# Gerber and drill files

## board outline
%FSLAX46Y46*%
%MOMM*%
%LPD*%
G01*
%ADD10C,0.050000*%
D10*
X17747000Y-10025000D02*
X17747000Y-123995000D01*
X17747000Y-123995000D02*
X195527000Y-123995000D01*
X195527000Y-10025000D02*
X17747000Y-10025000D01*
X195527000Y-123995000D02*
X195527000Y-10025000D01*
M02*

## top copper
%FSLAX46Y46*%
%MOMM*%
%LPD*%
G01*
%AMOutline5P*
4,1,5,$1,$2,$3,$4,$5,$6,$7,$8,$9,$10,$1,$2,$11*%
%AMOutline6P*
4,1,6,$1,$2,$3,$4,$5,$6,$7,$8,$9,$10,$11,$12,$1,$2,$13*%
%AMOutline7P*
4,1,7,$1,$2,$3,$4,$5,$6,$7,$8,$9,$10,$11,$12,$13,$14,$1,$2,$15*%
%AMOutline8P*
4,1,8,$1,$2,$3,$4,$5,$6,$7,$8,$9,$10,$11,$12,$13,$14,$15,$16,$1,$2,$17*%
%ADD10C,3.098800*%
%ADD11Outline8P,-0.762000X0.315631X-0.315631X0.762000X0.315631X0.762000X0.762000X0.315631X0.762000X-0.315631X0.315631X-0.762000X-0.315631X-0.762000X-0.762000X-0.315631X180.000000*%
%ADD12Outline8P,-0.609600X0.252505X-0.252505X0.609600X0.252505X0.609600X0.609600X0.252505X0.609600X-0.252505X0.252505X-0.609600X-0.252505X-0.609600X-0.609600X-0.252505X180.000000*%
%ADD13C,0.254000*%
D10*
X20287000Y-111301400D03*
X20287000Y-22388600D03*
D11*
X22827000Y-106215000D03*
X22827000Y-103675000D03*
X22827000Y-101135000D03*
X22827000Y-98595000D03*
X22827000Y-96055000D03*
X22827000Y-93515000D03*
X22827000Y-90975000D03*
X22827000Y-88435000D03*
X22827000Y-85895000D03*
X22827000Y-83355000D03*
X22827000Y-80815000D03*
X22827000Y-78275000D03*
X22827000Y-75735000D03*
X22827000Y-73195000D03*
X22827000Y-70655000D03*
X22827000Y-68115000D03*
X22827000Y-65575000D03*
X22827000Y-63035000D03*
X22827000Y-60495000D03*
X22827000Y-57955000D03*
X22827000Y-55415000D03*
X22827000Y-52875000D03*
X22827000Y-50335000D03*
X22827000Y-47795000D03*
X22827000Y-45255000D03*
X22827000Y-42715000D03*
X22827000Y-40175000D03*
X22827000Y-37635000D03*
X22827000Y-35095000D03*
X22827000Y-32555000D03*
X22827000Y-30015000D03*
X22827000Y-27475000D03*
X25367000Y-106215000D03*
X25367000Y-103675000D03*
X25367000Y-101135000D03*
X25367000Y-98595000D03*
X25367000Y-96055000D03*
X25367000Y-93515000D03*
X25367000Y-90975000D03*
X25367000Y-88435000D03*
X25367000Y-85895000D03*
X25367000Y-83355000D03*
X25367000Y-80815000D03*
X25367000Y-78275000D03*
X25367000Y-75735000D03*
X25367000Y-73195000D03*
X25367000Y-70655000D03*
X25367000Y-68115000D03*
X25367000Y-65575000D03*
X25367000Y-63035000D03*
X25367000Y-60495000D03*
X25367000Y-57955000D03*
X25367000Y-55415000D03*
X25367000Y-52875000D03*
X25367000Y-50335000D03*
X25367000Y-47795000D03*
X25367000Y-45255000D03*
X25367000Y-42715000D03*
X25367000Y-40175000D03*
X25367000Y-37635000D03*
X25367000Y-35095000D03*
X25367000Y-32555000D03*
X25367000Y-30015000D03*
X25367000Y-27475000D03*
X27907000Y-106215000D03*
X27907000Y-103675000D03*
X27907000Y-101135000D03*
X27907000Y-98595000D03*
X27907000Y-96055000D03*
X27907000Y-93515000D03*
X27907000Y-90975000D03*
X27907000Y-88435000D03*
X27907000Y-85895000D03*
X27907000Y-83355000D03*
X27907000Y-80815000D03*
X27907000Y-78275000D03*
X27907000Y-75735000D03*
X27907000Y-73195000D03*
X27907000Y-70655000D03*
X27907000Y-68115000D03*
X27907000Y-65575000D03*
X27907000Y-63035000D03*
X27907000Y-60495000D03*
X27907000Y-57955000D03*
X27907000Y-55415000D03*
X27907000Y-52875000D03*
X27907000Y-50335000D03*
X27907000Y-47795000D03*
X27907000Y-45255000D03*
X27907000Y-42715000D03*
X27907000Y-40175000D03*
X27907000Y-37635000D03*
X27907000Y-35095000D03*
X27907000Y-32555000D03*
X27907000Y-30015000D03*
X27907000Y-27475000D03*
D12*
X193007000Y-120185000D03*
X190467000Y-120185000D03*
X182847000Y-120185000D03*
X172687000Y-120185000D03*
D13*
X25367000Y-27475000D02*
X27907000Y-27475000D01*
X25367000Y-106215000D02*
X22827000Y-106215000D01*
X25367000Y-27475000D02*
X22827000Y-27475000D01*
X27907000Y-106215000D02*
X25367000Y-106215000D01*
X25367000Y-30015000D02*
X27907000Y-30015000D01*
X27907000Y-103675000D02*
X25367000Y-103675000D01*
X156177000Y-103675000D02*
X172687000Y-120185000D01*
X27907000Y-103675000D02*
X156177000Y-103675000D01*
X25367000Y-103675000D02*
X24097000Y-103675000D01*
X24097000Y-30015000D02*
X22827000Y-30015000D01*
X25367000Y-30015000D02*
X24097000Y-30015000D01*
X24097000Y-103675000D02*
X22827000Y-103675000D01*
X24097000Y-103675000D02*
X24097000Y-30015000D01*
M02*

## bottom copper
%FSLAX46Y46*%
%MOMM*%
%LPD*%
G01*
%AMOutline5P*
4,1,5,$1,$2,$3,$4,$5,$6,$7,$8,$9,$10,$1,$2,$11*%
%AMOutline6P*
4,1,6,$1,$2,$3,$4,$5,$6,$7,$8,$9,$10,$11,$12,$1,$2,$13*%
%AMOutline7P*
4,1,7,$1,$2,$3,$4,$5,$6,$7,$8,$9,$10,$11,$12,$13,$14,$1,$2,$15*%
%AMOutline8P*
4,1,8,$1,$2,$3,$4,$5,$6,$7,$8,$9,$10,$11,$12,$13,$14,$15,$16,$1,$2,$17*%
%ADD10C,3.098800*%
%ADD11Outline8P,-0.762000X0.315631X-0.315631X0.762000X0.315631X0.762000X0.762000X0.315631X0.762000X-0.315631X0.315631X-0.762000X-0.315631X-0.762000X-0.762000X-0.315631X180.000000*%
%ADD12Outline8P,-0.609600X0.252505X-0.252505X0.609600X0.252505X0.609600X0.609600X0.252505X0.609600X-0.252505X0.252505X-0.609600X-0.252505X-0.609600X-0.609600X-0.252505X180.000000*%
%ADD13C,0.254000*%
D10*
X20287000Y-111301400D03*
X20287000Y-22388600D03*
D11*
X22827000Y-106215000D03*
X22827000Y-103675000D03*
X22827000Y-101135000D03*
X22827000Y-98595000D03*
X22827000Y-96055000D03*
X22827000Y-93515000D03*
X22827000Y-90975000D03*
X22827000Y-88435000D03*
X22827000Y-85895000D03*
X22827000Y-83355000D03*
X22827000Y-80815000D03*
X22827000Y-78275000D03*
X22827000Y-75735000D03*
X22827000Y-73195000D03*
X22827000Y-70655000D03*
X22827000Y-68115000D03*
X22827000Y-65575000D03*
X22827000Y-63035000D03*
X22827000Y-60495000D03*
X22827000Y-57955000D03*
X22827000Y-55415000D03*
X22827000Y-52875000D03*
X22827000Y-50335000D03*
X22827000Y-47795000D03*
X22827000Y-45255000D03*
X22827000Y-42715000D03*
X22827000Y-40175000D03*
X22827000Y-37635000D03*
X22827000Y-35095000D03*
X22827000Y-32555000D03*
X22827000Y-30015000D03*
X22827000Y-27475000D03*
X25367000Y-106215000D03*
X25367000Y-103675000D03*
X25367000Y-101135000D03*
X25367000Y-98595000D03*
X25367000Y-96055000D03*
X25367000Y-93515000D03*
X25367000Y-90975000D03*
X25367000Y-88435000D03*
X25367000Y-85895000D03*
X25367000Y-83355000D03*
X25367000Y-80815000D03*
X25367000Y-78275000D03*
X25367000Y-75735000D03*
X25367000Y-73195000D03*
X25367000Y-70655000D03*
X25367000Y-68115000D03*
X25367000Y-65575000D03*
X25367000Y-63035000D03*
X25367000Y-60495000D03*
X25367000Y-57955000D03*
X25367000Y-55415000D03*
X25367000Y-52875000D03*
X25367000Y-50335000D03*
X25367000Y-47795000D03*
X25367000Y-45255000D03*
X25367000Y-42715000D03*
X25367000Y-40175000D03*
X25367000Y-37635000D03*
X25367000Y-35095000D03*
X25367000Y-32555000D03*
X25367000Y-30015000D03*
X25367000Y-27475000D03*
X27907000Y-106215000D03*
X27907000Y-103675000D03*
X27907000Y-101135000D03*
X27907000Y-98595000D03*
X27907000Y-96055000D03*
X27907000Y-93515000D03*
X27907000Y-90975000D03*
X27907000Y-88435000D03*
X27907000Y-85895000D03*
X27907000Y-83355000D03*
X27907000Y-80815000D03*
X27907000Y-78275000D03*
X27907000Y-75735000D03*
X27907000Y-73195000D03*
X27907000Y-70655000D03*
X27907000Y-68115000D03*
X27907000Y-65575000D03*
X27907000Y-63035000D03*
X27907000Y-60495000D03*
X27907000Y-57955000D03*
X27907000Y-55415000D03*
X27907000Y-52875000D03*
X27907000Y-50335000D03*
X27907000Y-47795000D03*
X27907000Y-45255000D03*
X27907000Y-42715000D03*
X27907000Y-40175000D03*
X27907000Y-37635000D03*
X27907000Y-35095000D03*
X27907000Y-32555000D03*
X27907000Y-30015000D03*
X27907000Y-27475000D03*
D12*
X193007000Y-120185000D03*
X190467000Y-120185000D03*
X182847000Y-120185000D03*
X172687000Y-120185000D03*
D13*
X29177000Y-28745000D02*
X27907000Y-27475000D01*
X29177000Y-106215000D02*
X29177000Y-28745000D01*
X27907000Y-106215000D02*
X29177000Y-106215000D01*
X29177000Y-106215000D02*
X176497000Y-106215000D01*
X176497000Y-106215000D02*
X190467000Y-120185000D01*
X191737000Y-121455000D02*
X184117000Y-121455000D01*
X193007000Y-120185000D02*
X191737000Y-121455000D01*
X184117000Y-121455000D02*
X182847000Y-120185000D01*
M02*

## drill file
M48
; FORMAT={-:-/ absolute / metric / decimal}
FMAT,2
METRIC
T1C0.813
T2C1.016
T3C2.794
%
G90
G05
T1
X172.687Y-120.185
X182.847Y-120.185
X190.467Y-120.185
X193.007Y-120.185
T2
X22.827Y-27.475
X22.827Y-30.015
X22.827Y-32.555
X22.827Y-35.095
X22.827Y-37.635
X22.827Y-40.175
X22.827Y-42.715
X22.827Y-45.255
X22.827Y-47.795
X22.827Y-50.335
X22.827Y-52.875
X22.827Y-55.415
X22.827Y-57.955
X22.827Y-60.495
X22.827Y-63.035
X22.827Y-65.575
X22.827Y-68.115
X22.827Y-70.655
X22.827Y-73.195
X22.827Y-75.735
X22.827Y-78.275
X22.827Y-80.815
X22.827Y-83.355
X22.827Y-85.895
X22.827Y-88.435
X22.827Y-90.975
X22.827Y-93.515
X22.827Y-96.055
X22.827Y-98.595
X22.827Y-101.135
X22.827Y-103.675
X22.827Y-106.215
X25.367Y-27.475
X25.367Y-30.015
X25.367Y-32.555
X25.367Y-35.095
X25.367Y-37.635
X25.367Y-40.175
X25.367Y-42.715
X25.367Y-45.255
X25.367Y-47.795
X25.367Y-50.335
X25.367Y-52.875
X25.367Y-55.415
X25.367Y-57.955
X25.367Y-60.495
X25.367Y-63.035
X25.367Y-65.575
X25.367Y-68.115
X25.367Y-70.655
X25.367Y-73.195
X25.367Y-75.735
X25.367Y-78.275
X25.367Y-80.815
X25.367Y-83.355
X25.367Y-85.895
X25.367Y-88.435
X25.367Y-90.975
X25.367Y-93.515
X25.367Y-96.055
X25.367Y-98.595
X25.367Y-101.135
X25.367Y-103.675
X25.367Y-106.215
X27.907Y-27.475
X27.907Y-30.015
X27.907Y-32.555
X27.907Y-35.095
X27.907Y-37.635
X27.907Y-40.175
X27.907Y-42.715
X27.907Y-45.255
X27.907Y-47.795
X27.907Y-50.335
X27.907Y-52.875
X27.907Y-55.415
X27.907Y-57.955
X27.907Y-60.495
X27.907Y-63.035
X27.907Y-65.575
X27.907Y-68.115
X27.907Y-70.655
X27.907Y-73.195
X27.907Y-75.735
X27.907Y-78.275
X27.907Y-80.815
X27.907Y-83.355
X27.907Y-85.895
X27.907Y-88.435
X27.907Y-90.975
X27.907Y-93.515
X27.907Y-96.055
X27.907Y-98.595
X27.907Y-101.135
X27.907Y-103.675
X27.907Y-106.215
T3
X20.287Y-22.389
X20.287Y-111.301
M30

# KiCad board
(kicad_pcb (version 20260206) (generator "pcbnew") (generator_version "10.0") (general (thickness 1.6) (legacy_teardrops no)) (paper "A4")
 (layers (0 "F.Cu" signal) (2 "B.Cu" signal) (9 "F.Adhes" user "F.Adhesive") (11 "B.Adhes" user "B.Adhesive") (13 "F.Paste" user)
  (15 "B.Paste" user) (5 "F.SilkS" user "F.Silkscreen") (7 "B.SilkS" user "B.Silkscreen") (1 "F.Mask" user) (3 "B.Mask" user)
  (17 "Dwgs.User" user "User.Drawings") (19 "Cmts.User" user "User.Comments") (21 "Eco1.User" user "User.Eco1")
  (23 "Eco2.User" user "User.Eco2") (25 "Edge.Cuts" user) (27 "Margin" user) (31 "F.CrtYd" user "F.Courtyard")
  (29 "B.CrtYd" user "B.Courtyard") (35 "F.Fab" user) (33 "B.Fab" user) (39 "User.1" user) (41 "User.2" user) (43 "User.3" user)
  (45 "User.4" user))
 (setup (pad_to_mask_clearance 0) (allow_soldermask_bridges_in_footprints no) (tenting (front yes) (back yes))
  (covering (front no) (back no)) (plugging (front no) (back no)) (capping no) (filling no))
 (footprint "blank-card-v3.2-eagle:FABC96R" (layer "F.Cu") (at 20.287 66.845 180)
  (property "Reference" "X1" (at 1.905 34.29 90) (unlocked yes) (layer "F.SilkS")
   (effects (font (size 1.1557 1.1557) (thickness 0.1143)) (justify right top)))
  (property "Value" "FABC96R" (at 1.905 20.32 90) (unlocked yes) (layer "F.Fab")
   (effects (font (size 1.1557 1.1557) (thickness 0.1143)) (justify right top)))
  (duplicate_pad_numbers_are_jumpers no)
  (pad "" np_thru_hole circle (at 0 -44.4564 180) (size 3.0988 3.0988) (drill 2.794) (layers "*.Cu" "*.Mask"))
  (pad "" np_thru_hole circle (at 0 44.4564 180) (size 3.0988 3.0988) (drill 2.794) (layers "*.Cu" "*.Mask"))
  (pad "A1" thru_hole roundrect (at -2.54 -39.37 180) (size 1.524 1.524) (drill 1.016) (layers "*.Cu" "*.Mask") (remove_unused_layers no)
   (roundrect_rratio 0.25) (chamfer_ratio 0.2928932188) (chamfer top_left top_right bottom_left bottom_right) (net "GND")
   (solder_mask_margin 0.0635) (thermal_bridge_angle 0))
  (pad "A2" thru_hole roundrect (at -2.54 -36.83 180) (size 1.524 1.524) (drill 1.016) (layers "*.Cu" "*.Mask") (remove_unused_layers no)
   (roundrect_rratio 0.25) (chamfer_ratio 0.2928932188) (chamfer top_left top_right bottom_left bottom_right) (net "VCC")
   (solder_mask_margin 0.0635) (thermal_bridge_angle 0))
  (pad "A3" thru_hole roundrect (at -2.54 -34.29 180) (size 1.524 1.524) (drill 1.016) (layers "*.Cu" "*.Mask") (remove_unused_layers no)
   (roundrect_rratio 0.25) (chamfer_ratio 0.2928932188) (chamfer top_left top_right bottom_left bottom_right) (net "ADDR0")
   (solder_mask_margin 0.0635) (thermal_bridge_angle 0))
  (pad "A4" thru_hole roundrect (at -2.54 -31.75 180) (size 1.524 1.524) (drill 1.016) (layers "*.Cu" "*.Mask") (remove_unused_layers no)
   (roundrect_rratio 0.25) (chamfer_ratio 0.2928932188) (chamfer top_left top_right bottom_left bottom_right) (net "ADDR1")
   (solder_mask_margin 0.0635) (thermal_bridge_angle 0))
  (pad "A5" thru_hole roundrect (at -2.54 -29.21 180) (size 1.524 1.524) (drill 1.016) (layers "*.Cu" "*.Mask") (remove_unused_layers no)
   (roundrect_rratio 0.25) (chamfer_ratio 0.2928932188) (chamfer top_left top_right bottom_left bottom_right) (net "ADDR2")
   (solder_mask_margin 0.0635) (thermal_bridge_angle 0))
  (pad "A6" thru_hole roundrect (at -2.54 -26.67 180) (size 1.524 1.524) (drill 1.016) (layers "*.Cu" "*.Mask") (remove_unused_layers no)
   (roundrect_rratio 0.25) (chamfer_ratio 0.2928932188) (chamfer top_left top_right bottom_left bottom_right) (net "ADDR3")
   (solder_mask_margin 0.0635) (thermal_bridge_angle 0))
  (pad "A7" thru_hole roundrect (at -2.54 -24.13 180) (size 1.524 1.524) (drill 1.016) (layers "*.Cu" "*.Mask") (remove_unused_layers no)
   (roundrect_rratio 0.25) (chamfer_ratio 0.2928932188) (chamfer top_left top_right bottom_left bottom_right) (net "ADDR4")
   (solder_mask_margin 0.0635) (thermal_bridge_angle 0))
  (pad "A8" thru_hole roundrect (at -2.54 -21.59 180) (size 1.524 1.524) (drill 1.016) (layers "*.Cu" "*.Mask") (remove_unused_layers no)
   (roundrect_rratio 0.25) (chamfer_ratio 0.2928932188) (chamfer top_left top_right bottom_left bottom_right) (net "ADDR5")
   (solder_mask_margin 0.0635) (thermal_bridge_angle 0))
  (pad "A9" thru_hole roundrect (at -2.54 -19.05 180) (size 1.524 1.524) (drill 1.016) (layers "*.Cu" "*.Mask") (remove_unused_layers no)
   (roundrect_rratio 0.25) (chamfer_ratio 0.2928932188) (chamfer top_left top_right bottom_left bottom_right) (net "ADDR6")
   (solder_mask_margin 0.0635) (thermal_bridge_angle 0))
  (pad "A10" thru_hole roundrect (at -2.54 -16.51 180) (size 1.524 1.524) (drill 1.016) (layers "*.Cu" "*.Mask") (remove_unused_layers no)
   (roundrect_rratio 0.25) (chamfer_ratio 0.2928932188) (chamfer top_left top_right bottom_left bottom_right) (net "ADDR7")
   (solder_mask_margin 0.0635) (thermal_bridge_angle 0))
  (pad "A11" thru_hole roundrect (at -2.54 -13.97 180) (size 1.524 1.524) (drill 1.016) (layers "*.Cu" "*.Mask") (remove_unused_layers no)
   (roundrect_rratio 0.25) (chamfer_ratio 0.2928932188) (chamfer top_left top_right bottom_left bottom_right) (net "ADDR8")
   (solder_mask_margin 0.0635) (thermal_bridge_angle 0))
  (pad "A12" thru_hole roundrect (at -2.54 -11.43 180) (size 1.524 1.524) (drill 1.016) (layers "*.Cu" "*.Mask") (remove_unused_layers no)
   (roundrect_rratio 0.25) (chamfer_ratio 0.2928932188) (chamfer top_left top_right bottom_left bottom_right) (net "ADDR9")
   (solder_mask_margin 0.0635) (thermal_bridge_angle 0))
  (pad "A13" thru_hole roundrect (at -2.54 -8.89 180) (size 1.524 1.524) (drill 1.016) (layers "*.Cu" "*.Mask") (remove_unused_layers no)
   (roundrect_rratio 0.25) (chamfer_ratio 0.2928932188) (chamfer top_left top_right bottom_left bottom_right) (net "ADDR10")
   (solder_mask_margin 0.0635) (thermal_bridge_angle 0))
  (pad "A14" thru_hole roundrect (at -2.54 -6.35 180) (size 1.524 1.524) (drill 1.016) (layers "*.Cu" "*.Mask") (remove_unused_layers no)
   (roundrect_rratio 0.25) (chamfer_ratio 0.2928932188) (chamfer top_left top_right bottom_left bottom_right) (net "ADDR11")
   (solder_mask_margin 0.0635) (thermal_bridge_angle 0))
  (pad "A15" thru_hole roundrect (at -2.54 -3.81 180) (size 1.524 1.524) (drill 1.016) (layers "*.Cu" "*.Mask") (remove_unused_layers no)
   (roundrect_rratio 0.25) (chamfer_ratio 0.2928932188) (chamfer top_left top_right bottom_left bottom_right) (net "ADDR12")
   (solder_mask_margin 0.0635) (thermal_bridge_angle 0))
  (pad "A16" thru_hole roundrect (at -2.54 -1.27 180) (size 1.524 1.524) (drill 1.016) (layers "*.Cu" "*.Mask") (remove_unused_layers no)
   (roundrect_rratio 0.25) (chamfer_ratio 0.2928932188) (chamfer top_left top_right bottom_left bottom_right) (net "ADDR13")
   (solder_mask_margin 0.0635) (thermal_bridge_angle 0))
  (pad "A17" thru_hole roundrect (at -2.54 1.27 180) (size 1.524 1.524) (drill 1.016) (layers "*.Cu" "*.Mask") (remove_unused_layers no)
   (roundrect_rratio 0.25) (chamfer_ratio 0.2928932188) (chamfer top_left top_right bottom_left bottom_right) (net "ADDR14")
   (solder_mask_margin 0.0635) (thermal_bridge_angle 0))
  (pad "A18" thru_hole roundrect (at -2.54 3.81 180) (size 1.524 1.524) (drill 1.016) (layers "*.Cu" "*.Mask") (remove_unused_layers no)
   (roundrect_rratio 0.25) (chamfer_ratio 0.2928932188) (chamfer top_left top_right bottom_left bottom_right) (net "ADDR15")
   (solder_mask_margin 0.0635) (thermal_bridge_angle 0))
  (pad "A19" thru_hole roundrect (at -2.54 6.35 180) (size 1.524 1.524) (drill 1.016) (layers "*.Cu" "*.Mask") (remove_unused_layers no)
   (roundrect_rratio 0.25) (chamfer_ratio 0.2928932188) (chamfer top_left top_right bottom_left bottom_right) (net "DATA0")
   (solder_mask_margin 0.0635) (thermal_bridge_angle 0))
  (pad "A20" thru_hole roundrect (at -2.54 8.89 180) (size 1.524 1.524) (drill 1.016) (layers "*.Cu" "*.Mask") (remove_unused_layers no)
   (roundrect_rratio 0.25) (chamfer_ratio 0.2928932188) (chamfer top_left top_right bottom_left bottom_right) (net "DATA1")
   (solder_mask_margin 0.0635) (thermal_bridge_angle 0))
  (pad "A21" thru_hole roundrect (at -2.54 11.43 180) (size 1.524 1.524) (drill 1.016) (layers "*.Cu" "*.Mask") (remove_unused_layers no)
   (roundrect_rratio 0.25) (chamfer_ratio 0.2928932188) (chamfer top_left top_right bottom_left bottom_right) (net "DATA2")
   (solder_mask_margin 0.0635) (thermal_bridge_angle 0))
  (pad "A22" thru_hole roundrect (at -2.54 13.97 180) (size 1.524 1.524) (drill 1.016) (layers "*.Cu" "*.Mask") (remove_unused_layers no)
   (roundrect_rratio 0.25) (chamfer_ratio 0.2928932188) (chamfer top_left top_right bottom_left bottom_right) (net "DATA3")
   (solder_mask_margin 0.0635) (thermal_bridge_angle 0))
  (pad "A23" thru_hole roundrect (at -2.54 16.51 180) (size 1.524 1.524) (drill 1.016) (layers "*.Cu" "*.Mask") (remove_unused_layers no)
   (roundrect_rratio 0.25) (chamfer_ratio 0.2928932188) (chamfer top_left top_right bottom_left bottom_right) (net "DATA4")
   (solder_mask_margin 0.0635) (thermal_bridge_angle 0))
  (pad "A24" thru_hole roundrect (at -2.54 19.05 180) (size 1.524 1.524) (drill 1.016) (layers "*.Cu" "*.Mask") (remove_unused_layers no)
   (roundrect_rratio 0.25) (chamfer_ratio 0.2928932188) (chamfer top_left top_right bottom_left bottom_right) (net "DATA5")
   (solder_mask_margin 0.0635) (thermal_bridge_angle 0))
  (pad "A25" thru_hole roundrect (at -2.54 21.59 180) (size 1.524 1.524) (drill 1.016) (layers "*.Cu" "*.Mask") (remove_unused_layers no)
   (roundrect_rratio 0.25) (chamfer_ratio 0.2928932188) (chamfer top_left top_right bottom_left bottom_right) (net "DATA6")
   (solder_mask_margin 0.0635) (thermal_bridge_angle 0))
  (pad "A26" thru_hole roundrect (at -2.54 24.13 180) (size 1.524 1.524) (drill 1.016) (layers "*.Cu" "*.Mask") (remove_unused_layers no)
   (roundrect_rratio 0.25) (chamfer_ratio 0.2928932188) (chamfer top_left top_right bottom_left bottom_right) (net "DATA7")
   (solder_mask_margin 0.0635) (thermal_bridge_angle 0))
  (pad "A27" thru_hole roundrect (at -2.54 26.67 180) (size 1.524 1.524) (drill 1.016) (layers "*.Cu" "*.Mask") (remove_unused_layers no)
   (roundrect_rratio 0.25) (chamfer_ratio 0.2928932188) (chamfer top_left top_right bottom_left bottom_right) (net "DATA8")
   (solder_mask_margin 0.0635) (thermal_bridge_angle 0))
  (pad "A28" thru_hole roundrect (at -2.54 29.21 180) (size 1.524 1.524) (drill 1.016) (layers "*.Cu" "*.Mask") (remove_unused_layers no)
   (roundrect_rratio 0.25) (chamfer_ratio 0.2928932188) (chamfer top_left top_right bottom_left bottom_right) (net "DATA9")
   (solder_mask_margin 0.0635) (thermal_bridge_angle 0))
  (pad "A29" thru_hole roundrect (at -2.54 31.75 180) (size 1.524 1.524) (drill 1.016) (layers "*.Cu" "*.Mask") (remove_unused_layers no)
   (roundrect_rratio 0.25) (chamfer_ratio 0.2928932188) (chamfer top_left top_right bottom_left bottom_right) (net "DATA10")
   (solder_mask_margin 0.0635) (thermal_bridge_angle 0))
  (pad "A30" thru_hole roundrect (at -2.54 34.29 180) (size 1.524 1.524) (drill 1.016) (layers "*.Cu" "*.Mask") (remove_unused_layers no)
   (roundrect_rratio 0.25) (chamfer_ratio 0.2928932188) (chamfer top_left top_right bottom_left bottom_right) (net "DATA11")
   (solder_mask_margin 0.0635) (thermal_bridge_angle 0))
  (pad "A31" thru_hole roundrect (at -2.54 36.83 180) (size 1.524 1.524) (drill 1.016) (layers "*.Cu" "*.Mask") (remove_unused_layers no)
   (roundrect_rratio 0.25) (chamfer_ratio 0.2928932188) (chamfer top_left top_right bottom_left bottom_right) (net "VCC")
   (solder_mask_margin 0.0635) (thermal_bridge_angle 0))
  (pad "A32" thru_hole roundrect (at -2.54 39.37 180) (size 1.524 1.524) (drill 1.016) (layers "*.Cu" "*.Mask") (remove_unused_layers no)
   (roundrect_rratio 0.25) (chamfer_ratio 0.2928932188) (chamfer top_left top_right bottom_left bottom_right) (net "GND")
   (solder_mask_margin 0.0635) (thermal_bridge_angle 0))
  (pad "B1" thru_hole roundrect (at -5.08 -39.37 180) (size 1.524 1.524) (drill 1.016) (layers "*.Cu" "*.Mask") (remove_unused_layers no)
   (roundrect_rratio 0.25) (chamfer_ratio 0.2928932188) (chamfer top_left top_right bottom_left bottom_right) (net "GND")
   (solder_mask_margin 0.0635) (thermal_bridge_angle 0))
  (pad "B2" thru_hole roundrect (at -5.08 -36.83 180) (size 1.524 1.524) (drill 1.016) (layers "*.Cu" "*.Mask") (remove_unused_layers no)
   (roundrect_rratio 0.25) (chamfer_ratio 0.2928932188) (chamfer top_left top_right bottom_left bottom_right) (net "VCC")
   (solder_mask_margin 0.0635) (thermal_bridge_angle 0))
  (pad "B3" thru_hole roundrect (at -5.08 -34.29 180) (size 1.524 1.524) (drill 1.016) (layers "*.Cu" "*.Mask") (remove_unused_layers no)
   (roundrect_rratio 0.25) (chamfer_ratio 0.2928932188) (chamfer top_left top_right bottom_left bottom_right) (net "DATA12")
   (solder_mask_margin 0.0635) (thermal_bridge_angle 0))
  (pad "B4" thru_hole roundrect (at -5.08 -31.75 180) (size 1.524 1.524) (drill 1.016) (layers "*.Cu" "*.Mask") (remove_unused_layers no)
   (roundrect_rratio 0.25) (chamfer_ratio 0.2928932188) (chamfer top_left top_right bottom_left bottom_right) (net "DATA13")
   (solder_mask_margin 0.0635) (thermal_bridge_angle 0))
  (pad "B5" thru_hole roundrect (at -5.08 -29.21 180) (size 1.524 1.524) (drill 1.016) (layers "*.Cu" "*.Mask") (remove_unused_layers no)
   (roundrect_rratio 0.25) (chamfer_ratio 0.2928932188) (chamfer top_left top_right bottom_left bottom_right) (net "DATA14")
   (solder_mask_margin 0.0635) (thermal_bridge_angle 0))
  (pad "B6" thru_hole roundrect (at -5.08 -26.67 180) (size 1.524 1.524) (drill 1.016) (layers "*.Cu" "*.Mask") (remove_unused_layers no)
   (roundrect_rratio 0.25) (chamfer_ratio 0.2928932188) (chamfer top_left top_right bottom_left bottom_right) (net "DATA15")
   (solder_mask_margin 0.0635) (thermal_bridge_angle 0))
  (pad "B7" thru_hole roundrect (at -5.08 -24.13 180) (size 1.524 1.524) (drill 1.016) (layers "*.Cu" "*.Mask") (remove_unused_layers no)
   (roundrect_rratio 0.25) (chamfer_ratio 0.2928932188) (chamfer top_left top_right bottom_left bottom_right) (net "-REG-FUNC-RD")
   (solder_mask_margin 0.0635) (thermal_bridge_angle 0))
  (pad "B8" thru_hole roundrect (at -5.08 -21.59 180) (size 1.524 1.524) (drill 1.016) (layers "*.Cu" "*.Mask") (remove_unused_layers no)
   (roundrect_rratio 0.25) (chamfer_ratio 0.2928932188) (chamfer top_left top_right bottom_left bottom_right) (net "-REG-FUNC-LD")
   (solder_mask_margin 0.0635) (thermal_bridge_angle 0))
  (pad "B9" thru_hole roundrect (at -5.08 -19.05 180) (size 1.524 1.524) (drill 1.016) (layers "*.Cu" "*.Mask") (remove_unused_layers no)
   (roundrect_rratio 0.25) (chamfer_ratio 0.2928932188) (chamfer top_left top_right bottom_left bottom_right) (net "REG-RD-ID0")
   (solder_mask_margin 0.0635) (thermal_bridge_angle 0))
  (pad "B10" thru_hole roundrect (at -5.08 -16.51 180) (size 1.524 1.524) (drill 1.016) (layers "*.Cu" "*.Mask") (remove_unused_layers no)
   (roundrect_rratio 0.25) (chamfer_ratio 0.2928932188) (chamfer top_left top_right bottom_left bottom_right) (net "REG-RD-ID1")
   (solder_mask_margin 0.0635) (thermal_bridge_angle 0))
  (pad "B11" thru_hole roundrect (at -5.08 -13.97 180) (size 1.524 1.524) (drill 1.016) (layers "*.Cu" "*.Mask") (remove_unused_layers no)
   (roundrect_rratio 0.25) (chamfer_ratio 0.2928932188) (chamfer top_left top_right bottom_left bottom_right) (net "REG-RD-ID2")
   (solder_mask_margin 0.0635) (thermal_bridge_angle 0))
  (pad "B12" thru_hole roundrect (at -5.08 -11.43 180) (size 1.524 1.524) (drill 1.016) (layers "*.Cu" "*.Mask") (remove_unused_layers no)
   (roundrect_rratio 0.25) (chamfer_ratio 0.2928932188) (chamfer top_left top_right bottom_left bottom_right) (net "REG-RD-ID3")
   (solder_mask_margin 0.0635) (thermal_bridge_angle 0))
  (pad "B13" thru_hole roundrect (at -5.08 -8.89 180) (size 1.524 1.524) (drill 1.016) (layers "*.Cu" "*.Mask") (remove_unused_layers no)
   (roundrect_rratio 0.25) (chamfer_ratio 0.2928932188) (chamfer top_left top_right bottom_left bottom_right) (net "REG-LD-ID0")
   (solder_mask_margin 0.0635) (thermal_bridge_angle 0))
  (pad "B14" thru_hole roundrect (at -5.08 -6.35 180) (size 1.524 1.524) (drill 1.016) (layers "*.Cu" "*.Mask") (remove_unused_layers no)
   (roundrect_rratio 0.25) (chamfer_ratio 0.2928932188) (chamfer top_left top_right bottom_left bottom_right) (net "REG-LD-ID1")
   (solder_mask_margin 0.0635) (thermal_bridge_angle 0))
  (pad "B15" thru_hole roundrect (at -5.08 -3.81 180) (size 1.524 1.524) (drill 1.016) (layers "*.Cu" "*.Mask") (remove_unused_layers no)
   (roundrect_rratio 0.25) (chamfer_ratio 0.2928932188) (chamfer top_left top_right bottom_left bottom_right) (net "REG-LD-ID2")
   (solder_mask_margin 0.0635) (thermal_bridge_angle 0))
  (pad "B16" thru_hole roundrect (at -5.08 -1.27 180) (size 1.524 1.524) (drill 1.016) (layers "*.Cu" "*.Mask") (remove_unused_layers no)
   (roundrect_rratio 0.25) (chamfer_ratio 0.2928932188) (chamfer top_left top_right bottom_left bottom_right) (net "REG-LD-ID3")
   (solder_mask_margin 0.0635) (thermal_bridge_angle 0))
  (pad "B17" thru_hole roundrect (at -5.08 1.27 180) (size 1.524 1.524) (drill 1.016) (layers "*.Cu" "*.Mask") (remove_unused_layers no)
   (roundrect_rratio 0.25) (chamfer_ratio 0.2928932188) (chamfer top_left top_right bottom_left bottom_right) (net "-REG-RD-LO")
   (solder_mask_margin 0.0635) (thermal_bridge_angle 0))
  (pad "B18" thru_hole roundrect (at -5.08 3.81 180) (size 1.524 1.524) (drill 1.016) (layers "*.Cu" "*.Mask") (remove_unused_layers no)
   (roundrect_rratio 0.25) (chamfer_ratio 0.2928932188) (chamfer top_left top_right bottom_left bottom_right) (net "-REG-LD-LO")
   (solder_mask_margin 0.0635) (thermal_bridge_angle 0))
  (pad "B19" thru_hole roundrect (at -5.08 6.35 180) (size 1.524 1.524) (drill 1.016) (layers "*.Cu" "*.Mask") (remove_unused_layers no)
   (roundrect_rratio 0.25) (chamfer_ratio 0.2928932188) (chamfer top_left top_right bottom_left bottom_right) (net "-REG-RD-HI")
   (solder_mask_margin 0.0635) (thermal_bridge_angle 0))
  (pad "B20" thru_hole roundrect (at -5.08 8.89 180) (size 1.524 1.524) (drill 1.016) (layers "*.Cu" "*.Mask") (remove_unused_layers no)
   (roundrect_rratio 0.25) (chamfer_ratio 0.2928932188) (chamfer top_left top_right bottom_left bottom_right) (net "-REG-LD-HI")
   (solder_mask_margin 0.0635) (thermal_bridge_angle 0))
  (pad "B21" thru_hole roundrect (at -5.08 11.43 180) (size 1.524 1.524) (drill 1.016) (layers "*.Cu" "*.Mask") (remove_unused_layers no)
   (roundrect_rratio 0.25) (chamfer_ratio 0.2928932188) (chamfer top_left top_right bottom_left bottom_right) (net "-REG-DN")
   (solder_mask_margin 0.0635) (thermal_bridge_angle 0))
  (pad "B22" thru_hole roundrect (at -5.08 13.97 180) (size 1.524 1.524) (drill 1.016) (layers "*.Cu" "*.Mask") (remove_unused_layers no)
   (roundrect_rratio 0.25) (chamfer_ratio 0.2928932188) (chamfer top_left top_right bottom_left bottom_right) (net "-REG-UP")
   (solder_mask_margin 0.0635) (thermal_bridge_angle 0))
  (pad "B23" thru_hole roundrect (at -5.08 16.51 180) (size 1.524 1.524) (drill 1.016) (layers "*.Cu" "*.Mask") (remove_unused_layers no)
   (roundrect_rratio 0.25) (chamfer_ratio 0.2928932188) (chamfer top_left top_right bottom_left bottom_right) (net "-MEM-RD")
   (solder_mask_margin 0.0635) (thermal_bridge_angle 0))
  (pad "B24" thru_hole roundrect (at -5.08 19.05 180) (size 1.524 1.524) (drill 1.016) (layers "*.Cu" "*.Mask") (remove_unused_layers no)
   (roundrect_rratio 0.25) (chamfer_ratio 0.2928932188) (chamfer top_left top_right bottom_left bottom_right) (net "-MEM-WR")
   (solder_mask_margin 0.0635) (thermal_bridge_angle 0))
  (pad "B25" thru_hole roundrect (at -5.08 21.59 180) (size 1.524 1.524) (drill 1.016) (layers "*.Cu" "*.Mask") (remove_unused_layers no)
   (roundrect_rratio 0.25) (chamfer_ratio 0.2928932188) (chamfer top_left top_right bottom_left bottom_right) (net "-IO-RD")
   (solder_mask_margin 0.0635) (thermal_bridge_angle 0))
  (pad "B26" thru_hole roundrect (at -5.08 24.13 180) (size 1.524 1.524) (drill 1.016) (layers "*.Cu" "*.Mask") (remove_unused_layers no)
   (roundrect_rratio 0.25) (chamfer_ratio 0.2928932188) (chamfer top_left top_right bottom_left bottom_right) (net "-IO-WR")
   (solder_mask_margin 0.0635) (thermal_bridge_angle 0))
  (pad "B27" thru_hole roundrect (at -5.08 26.67 180) (size 1.524 1.524) (drill 1.016) (layers "*.Cu" "*.Mask") (remove_unused_layers no)
   (roundrect_rratio 0.25) (chamfer_ratio 0.2928932188) (chamfer top_left top_right bottom_left bottom_right) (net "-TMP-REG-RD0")
   (solder_mask_margin 0.0635) (thermal_bridge_angle 0))
  (pad "B28" thru_hole roundrect (at -5.08 29.21 180) (size 1.524 1.524) (drill 1.016) (layers "*.Cu" "*.Mask") (remove_unused_layers no)
   (roundrect_rratio 0.25) (chamfer_ratio 0.2928932188) (chamfer top_left top_right bottom_left bottom_right) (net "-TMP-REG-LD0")
   (solder_mask_margin 0.0635) (thermal_bridge_angle 0))
  (pad "B29" thru_hole roundrect (at -5.08 31.75 180) (size 1.524 1.524) (drill 1.016) (layers "*.Cu" "*.Mask") (remove_unused_layers no)
   (roundrect_rratio 0.25) (chamfer_ratio 0.2928932188) (chamfer top_left top_right bottom_left bottom_right) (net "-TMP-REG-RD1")
   (solder_mask_margin 0.0635) (thermal_bridge_angle 0))
  (pad "B30" thru_hole roundrect (at -5.08 34.29 180) (size 1.524 1.524) (drill 1.016) (layers "*.Cu" "*.Mask") (remove_unused_layers no)
   (roundrect_rratio 0.25) (chamfer_ratio 0.2928932188) (chamfer top_left top_right bottom_left bottom_right) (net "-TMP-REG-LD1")
   (solder_mask_margin 0.0635) (thermal_bridge_angle 0))
  (pad "B31" thru_hole roundrect (at -5.08 36.83 180) (size 1.524 1.524) (drill 1.016) (layers "*.Cu" "*.Mask") (remove_unused_layers no)
   (roundrect_rratio 0.25) (chamfer_ratio 0.2928932188) (chamfer top_left top_right bottom_left bottom_right) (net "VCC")
   (solder_mask_margin 0.0635) (thermal_bridge_angle 0))
  (pad "B32" thru_hole roundrect (at -5.08 39.37 180) (size 1.524 1.524) (drill 1.016) (layers "*.Cu" "*.Mask") (remove_unused_layers no)
   (roundrect_rratio 0.25) (chamfer_ratio 0.2928932188) (chamfer top_left top_right bottom_left bottom_right) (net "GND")
   (solder_mask_margin 0.0635) (thermal_bridge_angle 0))
  (pad "C1" thru_hole roundrect (at -7.62 -39.37 180) (size 1.524 1.524) (drill 1.016) (layers "*.Cu" "*.Mask") (remove_unused_layers no)
   (roundrect_rratio 0.25) (chamfer_ratio 0.2928932188) (chamfer top_left top_right bottom_left bottom_right) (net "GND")
   (solder_mask_margin 0.0635) (thermal_bridge_angle 0))
  (pad "C2" thru_hole roundrect (at -7.62 -36.83 180) (size 1.524 1.524) (drill 1.016) (layers "*.Cu" "*.Mask") (remove_unused_layers no)
   (roundrect_rratio 0.25) (chamfer_ratio 0.2928932188) (chamfer top_left top_right bottom_left bottom_right) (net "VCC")
   (solder_mask_margin 0.0635) (thermal_bridge_angle 0))
  (pad "C3" thru_hole roundrect (at -7.62 -34.29 180) (size 1.524 1.524) (drill 1.016) (layers "*.Cu" "*.Mask") (remove_unused_layers no)
   (roundrect_rratio 0.25) (chamfer_ratio 0.2928932188) (chamfer top_left top_right bottom_left bottom_right) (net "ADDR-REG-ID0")
   (solder_mask_margin 0.0635) (thermal_bridge_angle 0))
  (pad "C4" thru_hole roundrect (at -7.62 -31.75 180) (size 1.524 1.524) (drill 1.016) (layers "*.Cu" "*.Mask") (remove_unused_layers no)
   (roundrect_rratio 0.25) (chamfer_ratio 0.2928932188) (chamfer top_left top_right bottom_left bottom_right) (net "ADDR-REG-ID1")
   (solder_mask_margin 0.0635) (thermal_bridge_angle 0))
  (pad "C5" thru_hole roundrect (at -7.62 -29.21 180) (size 1.524 1.524) (drill 1.016) (layers "*.Cu" "*.Mask") (remove_unused_layers no)
   (roundrect_rratio 0.25) (chamfer_ratio 0.2928932188) (chamfer top_left top_right bottom_left bottom_right) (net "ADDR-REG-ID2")
   (solder_mask_margin 0.0635) (thermal_bridge_angle 0))
  (pad "C6" thru_hole roundrect (at -7.62 -26.67 180) (size 1.524 1.524) (drill 1.016) (layers "*.Cu" "*.Mask") (remove_unused_layers no)
   (roundrect_rratio 0.25) (chamfer_ratio 0.2928932188) (chamfer top_left top_right bottom_left bottom_right) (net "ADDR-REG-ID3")
   (solder_mask_margin 0.0635) (thermal_bridge_angle 0))
  (pad "C7" thru_hole roundrect (at -7.62 -24.13 180) (size 1.524 1.524) (drill 1.016) (layers "*.Cu" "*.Mask") (remove_unused_layers no)
   (roundrect_rratio 0.25) (chamfer_ratio 0.2928932188) (chamfer top_left top_right bottom_left bottom_right) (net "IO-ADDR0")
   (solder_mask_margin 0.0635) (thermal_bridge_angle 0))
  (pad "C8" thru_hole roundrect (at -7.62 -21.59 180) (size 1.524 1.524) (drill 1.016) (layers "*.Cu" "*.Mask") (remove_unused_layers no)
   (roundrect_rratio 0.25) (chamfer_ratio 0.2928932188) (chamfer top_left top_right bottom_left bottom_right) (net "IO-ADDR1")
   (solder_mask_margin 0.0635) (thermal_bridge_angle 0))
  (pad "C9" thru_hole roundrect (at -7.62 -19.05 180) (size 1.524 1.524) (drill 1.016) (layers "*.Cu" "*.Mask") (remove_unused_layers no)
   (roundrect_rratio 0.25) (chamfer_ratio 0.2928932188) (chamfer top_left top_right bottom_left bottom_right) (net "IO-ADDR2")
   (solder_mask_margin 0.0635) (thermal_bridge_angle 0))
  (pad "C10" thru_hole roundrect (at -7.62 -16.51 180) (size 1.524 1.524) (drill 1.016) (layers "*.Cu" "*.Mask") (remove_unused_layers no)
   (roundrect_rratio 0.25) (chamfer_ratio 0.2928932188) (chamfer top_left top_right bottom_left bottom_right) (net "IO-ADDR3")
   (solder_mask_margin 0.0635) (thermal_bridge_angle 0))
  (pad "C11" thru_hole roundrect (at -7.62 -13.97 180) (size 1.524 1.524) (drill 1.016) (layers "*.Cu" "*.Mask") (remove_unused_layers no)
   (roundrect_rratio 0.25) (chamfer_ratio 0.2928932188) (chamfer top_left top_right bottom_left bottom_right) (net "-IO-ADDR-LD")
   (solder_mask_margin 0.0635) (thermal_bridge_angle 0))
  (pad "C12" thru_hole roundrect (at -7.62 -11.43 180) (size 1.524 1.524) (drill 1.016) (layers "*.Cu" "*.Mask") (remove_unused_layers no)
   (roundrect_rratio 0.25) (chamfer_ratio 0.2928932188) (chamfer top_left top_right bottom_left bottom_right) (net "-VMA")
   (solder_mask_margin 0.0635) (thermal_bridge_angle 0))
  (pad "C13" thru_hole roundrect (at -7.62 -8.89 180) (size 1.524 1.524) (drill 1.016) (layers "*.Cu" "*.Mask") (remove_unused_layers no)
   (roundrect_rratio 0.25) (chamfer_ratio 0.2928932188) (chamfer top_left top_right bottom_left bottom_right) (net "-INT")
   (solder_mask_margin 0.0635) (thermal_bridge_angle 0))
  (pad "C14" thru_hole roundrect (at -7.62 -6.35 180) (size 1.524 1.524) (drill 1.016) (layers "*.Cu" "*.Mask") (remove_unused_layers no)
   (roundrect_rratio 0.25) (chamfer_ratio 0.2928932188) (chamfer top_left top_right bottom_left bottom_right) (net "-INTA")
   (solder_mask_margin 0.0635) (thermal_bridge_angle 0))
  (pad "C15" thru_hole roundrect (at -7.62 -3.81 180) (size 1.524 1.524) (drill 1.016) (layers "*.Cu" "*.Mask") (remove_unused_layers no)
   (roundrect_rratio 0.25) (chamfer_ratio 0.2928932188) (chamfer top_left top_right bottom_left bottom_right) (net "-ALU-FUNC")
   (solder_mask_margin 0.0635) (thermal_bridge_angle 0))
  (pad "C16" thru_hole roundrect (at -7.62 -1.27 180) (size 1.524 1.524) (drill 1.016) (layers "*.Cu" "*.Mask") (remove_unused_layers no)
   (roundrect_rratio 0.25) (chamfer_ratio 0.2928932188) (chamfer top_left top_right bottom_left bottom_right) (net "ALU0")
   (solder_mask_margin 0.0635) (thermal_bridge_angle 0))
  (pad "C17" thru_hole roundrect (at -7.62 1.27 180) (size 1.524 1.524) (drill 1.016) (layers "*.Cu" "*.Mask") (remove_unused_layers no)
   (roundrect_rratio 0.25) (chamfer_ratio 0.2928932188) (chamfer top_left top_right bottom_left bottom_right) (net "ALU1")
   (solder_mask_margin 0.0635) (thermal_bridge_angle 0))
  (pad "C18" thru_hole roundrect (at -7.62 3.81 180) (size 1.524 1.524) (drill 1.016) (layers "*.Cu" "*.Mask") (remove_unused_layers no)
   (roundrect_rratio 0.25) (chamfer_ratio 0.2928932188) (chamfer top_left top_right bottom_left bottom_right) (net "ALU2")
   (solder_mask_margin 0.0635) (thermal_bridge_angle 0))
  (pad "C19" thru_hole roundrect (at -7.62 6.35 180) (size 1.524 1.524) (drill 1.016) (layers "*.Cu" "*.Mask") (remove_unused_layers no)
   (roundrect_rratio 0.25) (chamfer_ratio 0.2928932188) (chamfer top_left top_right bottom_left bottom_right) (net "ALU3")
   (solder_mask_margin 0.0635) (thermal_bridge_angle 0))
  (pad "C20" thru_hole roundrect (at -7.62 8.89 180) (size 1.524 1.524) (drill 1.016) (layers "*.Cu" "*.Mask") (remove_unused_layers no)
   (roundrect_rratio 0.25) (chamfer_ratio 0.2928932188) (chamfer top_left top_right bottom_left bottom_right) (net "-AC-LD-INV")
   (solder_mask_margin 0.0635) (thermal_bridge_angle 0))
  (pad "C21" thru_hole roundrect (at -7.62 11.43 180) (size 1.524 1.524) (drill 1.016) (layers "*.Cu" "*.Mask") (remove_unused_layers no)
   (roundrect_rratio 0.25) (chamfer_ratio 0.2928932188) (chamfer top_left top_right bottom_left bottom_right) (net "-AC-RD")
   (solder_mask_margin 0.0635) (thermal_bridge_angle 0))
  (pad "C22" thru_hole roundrect (at -7.62 13.97 180) (size 1.524 1.524) (drill 1.016) (layers "*.Cu" "*.Mask") (remove_unused_layers no)
   (roundrect_rratio 0.25) (chamfer_ratio 0.2928932188) (chamfer top_left top_right bottom_left bottom_right) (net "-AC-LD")
   (solder_mask_margin 0.0635) (thermal_bridge_angle 0))
  (pad "C23" thru_hole roundrect (at -7.62 16.51 180) (size 1.524 1.524) (drill 1.016) (layers "*.Cu" "*.Mask") (remove_unused_layers no)
   (roundrect_rratio 0.25) (chamfer_ratio 0.2928932188) (chamfer top_left top_right bottom_left bottom_right) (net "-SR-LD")
   (solder_mask_margin 0.0635) (thermal_bridge_angle 0))
  (pad "C24" thru_hole roundrect (at -7.62 19.05 180) (size 1.524 1.524) (drill 1.016) (layers "*.Cu" "*.Mask") (remove_unused_layers no)
   (roundrect_rratio 0.25) (chamfer_ratio 0.2928932188) (chamfer top_left top_right bottom_left bottom_right) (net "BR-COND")
   (solder_mask_margin 0.0635) (thermal_bridge_angle 0))
  (pad "C25" thru_hole roundrect (at -7.62 21.59 180) (size 1.524 1.524) (drill 1.016) (layers "*.Cu" "*.Mask") (remove_unused_layers no)
   (roundrect_rratio 0.25) (chamfer_ratio 0.2928932188) (chamfer top_left top_right bottom_left bottom_right) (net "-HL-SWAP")
   (solder_mask_margin 0.0635) (thermal_bridge_angle 0))
  (pad "C26" thru_hole roundrect (at -7.62 24.13 180) (size 1.524 1.524) (drill 1.016) (layers "*.Cu" "*.Mask") (remove_unused_layers no)
   (roundrect_rratio 0.25) (chamfer_ratio 0.2928932188) (chamfer top_left top_right bottom_left bottom_right) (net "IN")
   (solder_mask_margin 0.0635) (thermal_bridge_angle 0))
  (pad "C27" thru_hole roundrect (at -7.62 26.67 180) (size 1.524 1.524) (drill 1.016) (layers "*.Cu" "*.Mask") (remove_unused_layers no)
   (roundrect_rratio 0.25) (chamfer_ratio 0.2928932188) (chamfer top_left top_right bottom_left bottom_right) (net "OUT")
   (solder_mask_margin 0.0635) (thermal_bridge_angle 0))
  (pad "C28" thru_hole roundrect (at -7.62 29.21 180) (size 1.524 1.524) (drill 1.016) (layers "*.Cu" "*.Mask") (remove_unused_layers no)
   (roundrect_rratio 0.25) (chamfer_ratio 0.2928932188) (chamfer top_left top_right bottom_left bottom_right) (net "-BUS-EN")
   (solder_mask_margin 0.0635) (thermal_bridge_angle 0))
  (pad "C29" thru_hole roundrect (at -7.62 31.75 180) (size 1.524 1.524) (drill 1.016) (layers "*.Cu" "*.Mask") (remove_unused_layers no)
   (roundrect_rratio 0.25) (chamfer_ratio 0.2928932188) (chamfer top_left top_right bottom_left bottom_right) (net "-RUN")
   (solder_mask_margin 0.0635) (thermal_bridge_angle 0))
  (pad "C30" thru_hole roundrect (at -7.62 34.29 180) (size 1.524 1.524) (drill 1.016) (layers "*.Cu" "*.Mask") (remove_unused_layers no)
   (roundrect_rratio 0.25) (chamfer_ratio 0.2928932188) (chamfer top_left top_right bottom_left bottom_right) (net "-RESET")
   (solder_mask_margin 0.0635) (thermal_bridge_angle 0))
  (pad "C31" thru_hole roundrect (at -7.62 36.83 180) (size 1.524 1.524) (drill 1.016) (layers "*.Cu" "*.Mask") (remove_unused_layers no)
   (roundrect_rratio 0.25) (chamfer_ratio 0.2928932188) (chamfer top_left top_right bottom_left bottom_right) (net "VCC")
   (solder_mask_margin 0.0635) (thermal_bridge_angle 0))
  (pad "C32" thru_hole roundrect (at -7.62 39.37 180) (size 1.524 1.524) (drill 1.016) (layers "*.Cu" "*.Mask") (remove_unused_layers no)
   (roundrect_rratio 0.25) (chamfer_ratio 0.2928932188) (chamfer top_left top_right bottom_left bottom_right) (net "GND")
   (solder_mask_margin 0.0635) (thermal_bridge_angle 0))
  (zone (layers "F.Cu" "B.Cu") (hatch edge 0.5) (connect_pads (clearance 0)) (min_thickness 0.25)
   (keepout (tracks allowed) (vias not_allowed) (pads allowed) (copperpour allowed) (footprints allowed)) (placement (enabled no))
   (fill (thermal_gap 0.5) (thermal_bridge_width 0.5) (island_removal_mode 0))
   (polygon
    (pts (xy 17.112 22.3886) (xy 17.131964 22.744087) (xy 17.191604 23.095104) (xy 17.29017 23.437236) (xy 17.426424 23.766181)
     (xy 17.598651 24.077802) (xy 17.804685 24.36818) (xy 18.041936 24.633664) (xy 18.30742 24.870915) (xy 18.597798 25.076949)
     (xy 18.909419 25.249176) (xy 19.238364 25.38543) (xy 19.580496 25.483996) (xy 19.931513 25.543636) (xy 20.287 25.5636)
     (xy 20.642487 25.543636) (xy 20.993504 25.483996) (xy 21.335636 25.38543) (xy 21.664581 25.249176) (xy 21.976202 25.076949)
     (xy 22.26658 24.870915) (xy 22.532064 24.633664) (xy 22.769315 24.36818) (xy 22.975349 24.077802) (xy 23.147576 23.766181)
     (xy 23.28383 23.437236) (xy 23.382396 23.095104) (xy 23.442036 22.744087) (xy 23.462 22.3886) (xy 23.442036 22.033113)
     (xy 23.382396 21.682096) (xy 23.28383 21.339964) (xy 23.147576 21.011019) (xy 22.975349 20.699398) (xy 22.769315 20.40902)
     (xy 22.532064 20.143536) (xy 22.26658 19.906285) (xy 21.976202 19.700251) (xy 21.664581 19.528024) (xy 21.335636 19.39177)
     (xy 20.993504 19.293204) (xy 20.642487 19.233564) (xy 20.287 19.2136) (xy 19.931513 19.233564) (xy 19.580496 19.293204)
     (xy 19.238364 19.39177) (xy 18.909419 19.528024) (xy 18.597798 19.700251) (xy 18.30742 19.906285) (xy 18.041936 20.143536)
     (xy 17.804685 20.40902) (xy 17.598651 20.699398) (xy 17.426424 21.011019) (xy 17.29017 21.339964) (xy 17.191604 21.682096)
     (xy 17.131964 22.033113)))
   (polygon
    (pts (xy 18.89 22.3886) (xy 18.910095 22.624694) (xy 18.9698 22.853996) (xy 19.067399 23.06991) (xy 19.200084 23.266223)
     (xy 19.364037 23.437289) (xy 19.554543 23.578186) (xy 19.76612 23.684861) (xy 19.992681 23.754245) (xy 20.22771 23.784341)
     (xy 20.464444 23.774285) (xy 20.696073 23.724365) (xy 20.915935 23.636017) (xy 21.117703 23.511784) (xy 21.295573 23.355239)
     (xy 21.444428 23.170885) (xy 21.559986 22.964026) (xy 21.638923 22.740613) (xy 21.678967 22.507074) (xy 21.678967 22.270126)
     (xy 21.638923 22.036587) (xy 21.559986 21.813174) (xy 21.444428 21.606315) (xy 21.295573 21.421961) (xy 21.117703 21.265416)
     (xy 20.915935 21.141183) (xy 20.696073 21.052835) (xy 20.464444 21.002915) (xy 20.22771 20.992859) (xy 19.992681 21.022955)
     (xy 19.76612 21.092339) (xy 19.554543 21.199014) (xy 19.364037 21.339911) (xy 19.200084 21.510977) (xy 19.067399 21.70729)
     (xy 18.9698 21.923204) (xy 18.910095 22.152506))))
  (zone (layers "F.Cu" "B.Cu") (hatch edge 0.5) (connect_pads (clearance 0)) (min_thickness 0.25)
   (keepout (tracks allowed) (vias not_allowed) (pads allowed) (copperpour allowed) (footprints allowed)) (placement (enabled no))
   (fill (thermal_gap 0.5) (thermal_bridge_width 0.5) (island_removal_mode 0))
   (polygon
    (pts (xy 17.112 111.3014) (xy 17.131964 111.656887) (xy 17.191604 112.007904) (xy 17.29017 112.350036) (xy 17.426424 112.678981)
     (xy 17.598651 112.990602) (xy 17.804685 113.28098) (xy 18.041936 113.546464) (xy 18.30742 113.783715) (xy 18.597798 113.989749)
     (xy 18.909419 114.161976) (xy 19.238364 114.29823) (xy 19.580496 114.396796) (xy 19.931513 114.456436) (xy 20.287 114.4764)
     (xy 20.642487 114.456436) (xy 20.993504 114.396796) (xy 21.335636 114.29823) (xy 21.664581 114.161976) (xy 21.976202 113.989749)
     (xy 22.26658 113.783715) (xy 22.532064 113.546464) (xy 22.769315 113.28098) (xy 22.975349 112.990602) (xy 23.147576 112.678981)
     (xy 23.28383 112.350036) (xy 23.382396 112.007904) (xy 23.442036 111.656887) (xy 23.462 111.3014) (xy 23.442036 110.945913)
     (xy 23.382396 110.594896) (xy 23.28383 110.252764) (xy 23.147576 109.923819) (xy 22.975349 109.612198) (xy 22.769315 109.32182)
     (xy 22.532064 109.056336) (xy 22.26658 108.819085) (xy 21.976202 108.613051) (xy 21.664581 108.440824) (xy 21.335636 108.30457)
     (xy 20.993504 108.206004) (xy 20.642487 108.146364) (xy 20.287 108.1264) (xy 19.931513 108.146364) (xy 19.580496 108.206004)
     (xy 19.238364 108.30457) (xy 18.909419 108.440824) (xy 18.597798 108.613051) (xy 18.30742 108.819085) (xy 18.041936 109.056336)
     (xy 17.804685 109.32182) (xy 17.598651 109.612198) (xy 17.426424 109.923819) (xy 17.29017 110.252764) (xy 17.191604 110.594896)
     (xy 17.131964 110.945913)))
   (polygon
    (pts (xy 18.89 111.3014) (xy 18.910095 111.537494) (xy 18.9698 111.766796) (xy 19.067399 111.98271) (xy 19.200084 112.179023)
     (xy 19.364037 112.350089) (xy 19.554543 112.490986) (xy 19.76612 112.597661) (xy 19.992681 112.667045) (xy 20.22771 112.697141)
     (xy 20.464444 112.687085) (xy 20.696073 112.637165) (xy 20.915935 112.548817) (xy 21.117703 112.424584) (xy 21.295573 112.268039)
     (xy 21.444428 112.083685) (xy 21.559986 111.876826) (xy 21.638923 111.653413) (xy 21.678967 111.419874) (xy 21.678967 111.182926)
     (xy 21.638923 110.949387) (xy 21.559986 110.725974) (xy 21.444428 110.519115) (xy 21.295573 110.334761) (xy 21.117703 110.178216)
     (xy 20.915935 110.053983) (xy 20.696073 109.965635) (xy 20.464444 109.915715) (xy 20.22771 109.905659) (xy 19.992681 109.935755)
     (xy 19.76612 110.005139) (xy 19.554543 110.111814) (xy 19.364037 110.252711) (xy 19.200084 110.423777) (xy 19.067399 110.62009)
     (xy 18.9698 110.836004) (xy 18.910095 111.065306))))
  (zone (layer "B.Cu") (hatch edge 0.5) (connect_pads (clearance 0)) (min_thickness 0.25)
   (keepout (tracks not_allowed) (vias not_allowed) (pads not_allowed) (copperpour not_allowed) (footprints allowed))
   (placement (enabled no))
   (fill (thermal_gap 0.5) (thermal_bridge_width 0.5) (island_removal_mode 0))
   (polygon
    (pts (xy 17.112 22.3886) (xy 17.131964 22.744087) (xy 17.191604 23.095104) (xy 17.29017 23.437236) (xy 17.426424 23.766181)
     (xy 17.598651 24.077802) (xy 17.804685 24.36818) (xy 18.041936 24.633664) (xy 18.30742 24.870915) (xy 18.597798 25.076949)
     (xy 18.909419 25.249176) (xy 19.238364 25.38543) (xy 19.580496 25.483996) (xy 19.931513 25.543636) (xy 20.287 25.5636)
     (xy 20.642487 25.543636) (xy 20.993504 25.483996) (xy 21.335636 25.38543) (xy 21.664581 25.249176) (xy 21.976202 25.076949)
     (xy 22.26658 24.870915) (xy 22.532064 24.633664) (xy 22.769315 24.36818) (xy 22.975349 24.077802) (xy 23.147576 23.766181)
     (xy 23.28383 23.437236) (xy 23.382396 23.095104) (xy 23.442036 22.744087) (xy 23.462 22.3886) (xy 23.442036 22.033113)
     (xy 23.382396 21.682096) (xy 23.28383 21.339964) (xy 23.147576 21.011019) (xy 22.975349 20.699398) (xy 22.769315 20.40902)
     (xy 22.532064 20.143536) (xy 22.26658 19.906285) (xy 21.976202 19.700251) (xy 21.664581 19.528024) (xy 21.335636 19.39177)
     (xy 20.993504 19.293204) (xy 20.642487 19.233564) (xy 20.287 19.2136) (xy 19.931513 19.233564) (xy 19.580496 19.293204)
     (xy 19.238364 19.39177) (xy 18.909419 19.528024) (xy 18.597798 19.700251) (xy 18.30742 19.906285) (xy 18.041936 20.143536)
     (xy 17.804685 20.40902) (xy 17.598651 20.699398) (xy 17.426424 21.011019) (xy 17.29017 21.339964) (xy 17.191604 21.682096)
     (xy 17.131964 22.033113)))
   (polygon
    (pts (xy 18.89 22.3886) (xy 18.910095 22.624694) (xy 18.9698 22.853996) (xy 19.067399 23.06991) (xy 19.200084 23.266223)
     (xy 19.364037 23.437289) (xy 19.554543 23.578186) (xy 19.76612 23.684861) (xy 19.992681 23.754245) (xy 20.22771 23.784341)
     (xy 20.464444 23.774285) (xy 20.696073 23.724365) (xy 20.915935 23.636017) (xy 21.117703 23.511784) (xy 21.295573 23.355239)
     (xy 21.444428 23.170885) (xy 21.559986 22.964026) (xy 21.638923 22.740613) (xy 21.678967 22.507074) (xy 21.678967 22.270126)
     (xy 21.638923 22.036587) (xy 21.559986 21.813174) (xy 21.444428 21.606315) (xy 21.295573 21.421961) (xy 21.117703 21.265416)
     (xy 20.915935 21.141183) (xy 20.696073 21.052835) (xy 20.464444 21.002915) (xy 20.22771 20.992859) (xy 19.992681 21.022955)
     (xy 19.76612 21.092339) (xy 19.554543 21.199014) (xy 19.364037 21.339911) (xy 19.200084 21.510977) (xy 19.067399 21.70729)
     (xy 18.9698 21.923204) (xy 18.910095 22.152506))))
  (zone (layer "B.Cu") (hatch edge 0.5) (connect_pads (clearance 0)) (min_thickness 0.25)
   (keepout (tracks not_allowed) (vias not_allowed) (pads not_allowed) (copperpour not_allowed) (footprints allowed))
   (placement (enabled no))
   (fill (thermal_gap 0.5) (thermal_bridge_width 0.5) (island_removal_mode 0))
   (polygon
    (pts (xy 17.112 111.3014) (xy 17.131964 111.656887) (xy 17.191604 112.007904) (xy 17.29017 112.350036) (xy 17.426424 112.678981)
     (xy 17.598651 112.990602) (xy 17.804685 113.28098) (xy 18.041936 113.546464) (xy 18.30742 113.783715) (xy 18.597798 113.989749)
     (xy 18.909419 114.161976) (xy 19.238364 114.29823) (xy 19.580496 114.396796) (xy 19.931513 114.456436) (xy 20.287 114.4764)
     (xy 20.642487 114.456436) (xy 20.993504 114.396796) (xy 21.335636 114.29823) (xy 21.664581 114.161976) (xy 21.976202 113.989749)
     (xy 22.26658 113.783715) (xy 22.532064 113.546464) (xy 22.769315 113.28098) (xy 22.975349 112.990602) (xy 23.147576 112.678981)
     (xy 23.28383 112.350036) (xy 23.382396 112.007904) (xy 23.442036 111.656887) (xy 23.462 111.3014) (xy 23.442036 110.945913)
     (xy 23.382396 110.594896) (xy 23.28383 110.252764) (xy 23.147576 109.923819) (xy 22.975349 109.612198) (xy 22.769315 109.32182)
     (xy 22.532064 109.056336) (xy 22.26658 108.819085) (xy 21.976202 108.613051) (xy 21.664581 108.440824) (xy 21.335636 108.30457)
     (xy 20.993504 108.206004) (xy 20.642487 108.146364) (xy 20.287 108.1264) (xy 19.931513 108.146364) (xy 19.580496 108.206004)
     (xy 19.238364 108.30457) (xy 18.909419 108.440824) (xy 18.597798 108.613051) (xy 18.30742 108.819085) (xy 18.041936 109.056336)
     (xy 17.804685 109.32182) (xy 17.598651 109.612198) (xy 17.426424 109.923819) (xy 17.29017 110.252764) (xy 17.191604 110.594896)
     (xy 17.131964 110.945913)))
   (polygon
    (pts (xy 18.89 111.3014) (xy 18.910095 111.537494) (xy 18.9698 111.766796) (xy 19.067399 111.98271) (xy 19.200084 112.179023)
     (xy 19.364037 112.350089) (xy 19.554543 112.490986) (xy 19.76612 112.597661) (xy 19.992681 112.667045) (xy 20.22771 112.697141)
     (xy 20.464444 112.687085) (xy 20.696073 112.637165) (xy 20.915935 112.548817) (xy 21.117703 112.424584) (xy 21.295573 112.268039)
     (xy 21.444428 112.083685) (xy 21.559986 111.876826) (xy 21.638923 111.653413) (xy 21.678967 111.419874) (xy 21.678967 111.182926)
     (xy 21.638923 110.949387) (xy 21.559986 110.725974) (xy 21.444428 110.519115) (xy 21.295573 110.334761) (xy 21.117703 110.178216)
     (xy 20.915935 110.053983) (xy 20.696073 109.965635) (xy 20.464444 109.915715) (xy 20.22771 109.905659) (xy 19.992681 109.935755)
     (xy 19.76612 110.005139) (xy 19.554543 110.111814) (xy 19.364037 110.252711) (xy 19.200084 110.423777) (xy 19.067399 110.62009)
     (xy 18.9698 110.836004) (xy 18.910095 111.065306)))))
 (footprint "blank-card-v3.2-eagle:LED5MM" (layer "F.Cu") (at 191.737 120.185 180)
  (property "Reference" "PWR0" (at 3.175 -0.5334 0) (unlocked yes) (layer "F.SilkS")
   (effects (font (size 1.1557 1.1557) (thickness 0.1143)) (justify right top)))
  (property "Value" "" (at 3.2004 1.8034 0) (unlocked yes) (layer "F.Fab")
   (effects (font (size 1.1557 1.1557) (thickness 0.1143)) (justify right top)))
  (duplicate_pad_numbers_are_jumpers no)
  (pad "A" thru_hole roundrect (at -1.27 0 180) (size 1.2192 1.2192) (drill 0.8128) (layers "*.Cu" "*.Mask") (remove_unused_layers no)
   (roundrect_rratio 0.25) (chamfer_ratio 0.2928932188) (chamfer top_left top_right bottom_left bottom_right) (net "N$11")
   (solder_mask_margin 0.0635) (thermal_bridge_angle 0))
  (pad "K" thru_hole roundrect (at 1.27 0 180) (size 1.2192 1.2192) (drill 0.8128) (layers "*.Cu" "*.Mask") (remove_unused_layers no)
   (roundrect_rratio 0.25) (chamfer_ratio 0.2928932188) (chamfer top_left top_right bottom_left bottom_right) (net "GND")
   (solder_mask_margin 0.0635) (thermal_bridge_angle 0)))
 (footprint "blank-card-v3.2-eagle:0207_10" (layer "F.Cu") (at 177.767 120.185 180)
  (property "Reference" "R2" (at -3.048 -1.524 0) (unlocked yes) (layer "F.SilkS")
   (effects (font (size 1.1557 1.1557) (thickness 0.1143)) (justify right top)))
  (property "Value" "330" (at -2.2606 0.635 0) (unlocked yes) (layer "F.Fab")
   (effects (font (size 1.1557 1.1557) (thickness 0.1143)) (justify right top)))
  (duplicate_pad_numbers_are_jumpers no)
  (pad "1" thru_hole roundrect (at -5.08 0 180) (size 1.2192 1.2192) (drill 0.8128) (layers "*.Cu" "*.Mask") (remove_unused_layers no)
   (roundrect_rratio 0.25) (chamfer_ratio 0.2928932188) (chamfer top_left top_right bottom_left bottom_right) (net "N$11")
   (solder_mask_margin 0.0635) (thermal_bridge_angle 0))
  (pad "2" thru_hole roundrect (at 5.08 0 180) (size 1.2192 1.2192) (drill 0.8128) (layers "*.Cu" "*.Mask") (remove_unused_layers no)
   (roundrect_rratio 0.25) (chamfer_ratio 0.2928932188) (chamfer top_left top_right bottom_left bottom_right) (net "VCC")
   (solder_mask_margin 0.0635) (thermal_bridge_angle 0)))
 (gr_line (start 17.747 10.025) (end 17.747 123.995) (stroke (width 0.05) (type solid)) (layer "Edge.Cuts"))
 (gr_line (start 17.747 123.995) (end 195.527 123.995) (stroke (width 0.05) (type solid)) (layer "Edge.Cuts"))
 (gr_line (start 195.527 10.025) (end 17.747 10.025) (stroke (width 0.05) (type solid)) (layer "Edge.Cuts"))
 (gr_line (start 195.527 123.995) (end 195.527 10.025) (stroke (width 0.05) (type solid)) (layer "Edge.Cuts"))
 (segment (start 25.367 27.475) (end 27.907 27.475) (width 0.254) (layer "F.Cu") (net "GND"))
 (segment (start 25.367 106.215) (end 22.827 106.215) (width 0.254) (layer "F.Cu") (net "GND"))
 (segment (start 25.367 27.475) (end 22.827 27.475) (width 0.254) (layer "F.Cu") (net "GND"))
 (segment (start 27.907 106.215) (end 25.367 106.215) (width 0.254) (layer "F.Cu") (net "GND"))
 (segment (start 29.177 28.745) (end 27.907 27.475) (width 0.254) (layer "B.Cu") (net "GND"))
 (segment (start 29.177 106.215) (end 29.177 28.745) (width 0.254) (layer "B.Cu") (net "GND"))
 (segment (start 27.907 106.215) (end 29.177 106.215) (width 0.254) (layer "B.Cu") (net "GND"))
 (segment (start 29.177 106.215) (end 176.497 106.215) (width 0.254) (layer "B.Cu") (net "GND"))
 (segment (start 176.497 106.215) (end 190.467 120.185) (width 0.254) (layer "B.Cu") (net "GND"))
 (segment (start 25.367 30.015) (end 27.907 30.015) (width 0.254) (layer "F.Cu") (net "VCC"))
 (segment (start 27.907 103.675) (end 25.367 103.675) (width 0.254) (layer "F.Cu") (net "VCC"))
 (segment (start 156.177 103.675) (end 172.687 120.185) (width 0.254) (layer "F.Cu") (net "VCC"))
 (segment (start 27.907 103.675) (end 156.177 103.675) (width 0.254) (layer "F.Cu") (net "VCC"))
 (segment (start 25.367 103.675) (end 24.097 103.675) (width 0.254) (layer "F.Cu") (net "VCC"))
 (segment (start 24.097 30.015) (end 22.827 30.015) (width 0.254) (layer "F.Cu") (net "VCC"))
 (segment (start 25.367 30.015) (end 24.097 30.015) (width 0.254) (layer "F.Cu") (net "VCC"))
 (segment (start 24.097 103.675) (end 22.827 103.675) (width 0.254) (layer "F.Cu") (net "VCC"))
 (segment (start 24.097 103.675) (end 24.097 30.015) (width 0.254) (layer "F.Cu") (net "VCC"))
 (segment (start 191.737 121.455) (end 184.117 121.455) (width 0.254) (layer "B.Cu") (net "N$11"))
 (segment (start 193.007 120.185) (end 191.737 121.455) (width 0.254) (layer "B.Cu") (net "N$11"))
 (segment (start 184.117 121.455) (end 182.847 120.185) (width 0.254) (layer "B.Cu") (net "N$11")))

